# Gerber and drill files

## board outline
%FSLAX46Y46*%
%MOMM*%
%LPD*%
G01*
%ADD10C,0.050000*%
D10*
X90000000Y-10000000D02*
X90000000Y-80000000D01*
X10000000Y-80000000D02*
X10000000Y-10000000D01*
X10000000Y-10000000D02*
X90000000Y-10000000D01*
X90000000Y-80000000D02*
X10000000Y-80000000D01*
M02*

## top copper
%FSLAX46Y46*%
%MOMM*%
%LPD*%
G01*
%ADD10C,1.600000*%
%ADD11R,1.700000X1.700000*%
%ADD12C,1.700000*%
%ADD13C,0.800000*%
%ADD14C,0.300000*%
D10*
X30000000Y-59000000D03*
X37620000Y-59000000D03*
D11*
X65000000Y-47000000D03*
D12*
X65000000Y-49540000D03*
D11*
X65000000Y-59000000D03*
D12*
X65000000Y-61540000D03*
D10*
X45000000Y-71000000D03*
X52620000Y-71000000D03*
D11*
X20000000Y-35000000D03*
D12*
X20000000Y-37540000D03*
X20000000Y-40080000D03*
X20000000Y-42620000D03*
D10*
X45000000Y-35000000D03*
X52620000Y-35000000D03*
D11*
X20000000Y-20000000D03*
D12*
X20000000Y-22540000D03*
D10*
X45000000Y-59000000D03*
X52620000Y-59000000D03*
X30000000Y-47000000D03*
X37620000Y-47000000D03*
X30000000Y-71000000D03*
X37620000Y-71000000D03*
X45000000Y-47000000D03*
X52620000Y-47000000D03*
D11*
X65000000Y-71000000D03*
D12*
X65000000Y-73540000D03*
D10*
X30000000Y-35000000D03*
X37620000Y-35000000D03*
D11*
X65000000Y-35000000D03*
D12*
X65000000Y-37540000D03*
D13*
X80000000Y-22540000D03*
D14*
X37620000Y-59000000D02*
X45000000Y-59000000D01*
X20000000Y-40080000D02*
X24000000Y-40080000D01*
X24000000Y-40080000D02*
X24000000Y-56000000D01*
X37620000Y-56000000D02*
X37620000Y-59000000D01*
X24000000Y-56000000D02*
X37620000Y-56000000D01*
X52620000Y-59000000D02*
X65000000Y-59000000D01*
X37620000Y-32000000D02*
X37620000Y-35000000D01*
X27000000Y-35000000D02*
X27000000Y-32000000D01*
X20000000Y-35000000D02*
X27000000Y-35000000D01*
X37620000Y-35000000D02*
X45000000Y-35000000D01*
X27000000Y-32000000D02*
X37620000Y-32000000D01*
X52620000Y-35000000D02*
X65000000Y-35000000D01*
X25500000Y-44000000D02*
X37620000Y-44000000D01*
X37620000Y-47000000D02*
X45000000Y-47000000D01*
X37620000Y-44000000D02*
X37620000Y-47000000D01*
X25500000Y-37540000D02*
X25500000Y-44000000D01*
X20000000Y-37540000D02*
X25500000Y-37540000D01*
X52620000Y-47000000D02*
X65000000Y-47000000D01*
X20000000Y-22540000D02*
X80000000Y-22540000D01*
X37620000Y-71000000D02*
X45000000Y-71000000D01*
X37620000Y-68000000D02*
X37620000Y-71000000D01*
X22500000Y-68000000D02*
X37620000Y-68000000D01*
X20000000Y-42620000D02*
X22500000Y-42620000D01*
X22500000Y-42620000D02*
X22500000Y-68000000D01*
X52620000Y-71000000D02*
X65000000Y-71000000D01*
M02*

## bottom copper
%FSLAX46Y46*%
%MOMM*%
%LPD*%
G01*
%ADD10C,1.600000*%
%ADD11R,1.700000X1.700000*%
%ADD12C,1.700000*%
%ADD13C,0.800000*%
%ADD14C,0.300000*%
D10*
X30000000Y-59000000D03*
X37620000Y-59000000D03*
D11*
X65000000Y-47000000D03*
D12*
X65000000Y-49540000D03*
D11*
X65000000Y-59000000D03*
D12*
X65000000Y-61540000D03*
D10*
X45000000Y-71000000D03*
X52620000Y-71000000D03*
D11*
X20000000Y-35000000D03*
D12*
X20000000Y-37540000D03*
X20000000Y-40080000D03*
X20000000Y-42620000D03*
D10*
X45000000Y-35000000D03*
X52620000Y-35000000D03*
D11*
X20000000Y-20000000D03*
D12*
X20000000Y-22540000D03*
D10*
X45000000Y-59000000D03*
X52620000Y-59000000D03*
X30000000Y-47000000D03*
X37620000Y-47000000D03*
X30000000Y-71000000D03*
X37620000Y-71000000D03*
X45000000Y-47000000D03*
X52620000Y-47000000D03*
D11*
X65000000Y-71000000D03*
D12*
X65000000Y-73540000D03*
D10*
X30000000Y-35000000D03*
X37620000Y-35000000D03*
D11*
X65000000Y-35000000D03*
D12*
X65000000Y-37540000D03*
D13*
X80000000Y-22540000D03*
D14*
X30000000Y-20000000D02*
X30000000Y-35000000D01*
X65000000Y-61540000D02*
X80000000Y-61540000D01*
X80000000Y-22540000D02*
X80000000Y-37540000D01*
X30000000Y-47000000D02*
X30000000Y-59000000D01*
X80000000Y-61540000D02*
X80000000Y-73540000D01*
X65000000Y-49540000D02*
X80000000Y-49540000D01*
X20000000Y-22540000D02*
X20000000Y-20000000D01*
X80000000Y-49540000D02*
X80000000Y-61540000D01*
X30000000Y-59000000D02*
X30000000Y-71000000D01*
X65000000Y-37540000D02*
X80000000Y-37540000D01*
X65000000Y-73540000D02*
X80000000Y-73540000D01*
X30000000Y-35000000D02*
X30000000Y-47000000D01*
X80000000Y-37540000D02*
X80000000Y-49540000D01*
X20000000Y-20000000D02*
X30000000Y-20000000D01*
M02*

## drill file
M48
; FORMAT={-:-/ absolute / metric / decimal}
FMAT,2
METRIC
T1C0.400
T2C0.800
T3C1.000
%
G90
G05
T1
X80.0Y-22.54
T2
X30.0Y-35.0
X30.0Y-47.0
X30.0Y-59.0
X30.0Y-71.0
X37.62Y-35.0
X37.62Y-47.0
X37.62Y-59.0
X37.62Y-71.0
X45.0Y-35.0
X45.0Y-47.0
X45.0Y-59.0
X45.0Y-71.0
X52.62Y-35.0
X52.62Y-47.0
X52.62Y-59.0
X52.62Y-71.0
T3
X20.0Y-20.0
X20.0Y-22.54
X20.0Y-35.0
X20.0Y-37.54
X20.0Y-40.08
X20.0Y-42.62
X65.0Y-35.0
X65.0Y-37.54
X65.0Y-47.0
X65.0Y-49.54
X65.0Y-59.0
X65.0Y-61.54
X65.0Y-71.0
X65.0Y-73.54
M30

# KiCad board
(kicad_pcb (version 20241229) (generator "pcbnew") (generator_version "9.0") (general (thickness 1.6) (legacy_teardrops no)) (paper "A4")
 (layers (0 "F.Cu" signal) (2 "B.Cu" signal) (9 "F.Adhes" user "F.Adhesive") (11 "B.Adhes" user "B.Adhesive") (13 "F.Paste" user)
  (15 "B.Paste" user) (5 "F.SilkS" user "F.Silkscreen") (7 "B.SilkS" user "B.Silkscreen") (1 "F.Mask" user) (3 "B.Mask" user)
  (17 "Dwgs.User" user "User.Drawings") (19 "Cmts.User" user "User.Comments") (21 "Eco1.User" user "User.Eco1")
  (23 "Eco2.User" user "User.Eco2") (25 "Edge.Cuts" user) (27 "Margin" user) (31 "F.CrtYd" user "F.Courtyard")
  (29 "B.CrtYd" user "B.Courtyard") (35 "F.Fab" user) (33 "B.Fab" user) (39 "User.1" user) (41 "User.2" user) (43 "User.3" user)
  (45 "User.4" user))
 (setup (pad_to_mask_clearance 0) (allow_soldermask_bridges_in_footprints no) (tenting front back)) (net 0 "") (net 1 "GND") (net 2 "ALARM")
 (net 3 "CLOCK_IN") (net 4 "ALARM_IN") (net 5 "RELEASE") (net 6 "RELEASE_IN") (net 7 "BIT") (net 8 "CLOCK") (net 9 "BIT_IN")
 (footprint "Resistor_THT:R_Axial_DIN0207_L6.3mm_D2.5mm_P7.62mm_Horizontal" (layer "F.Cu") (at 30 59)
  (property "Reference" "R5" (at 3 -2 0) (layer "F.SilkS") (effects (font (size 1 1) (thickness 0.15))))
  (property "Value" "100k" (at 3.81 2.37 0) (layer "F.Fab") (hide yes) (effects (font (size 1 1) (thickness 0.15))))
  (pad "1" thru_hole circle (at 0 0) (size 1.6 1.6) (drill 0.8) (layers "*.Cu" "*.Mask") (remove_unused_layers no) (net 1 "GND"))
  (pad "2" thru_hole circle (at 7.62 0) (size 1.6 1.6) (drill 0.8) (layers "*.Cu" "*.Mask") (remove_unused_layers no) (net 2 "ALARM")))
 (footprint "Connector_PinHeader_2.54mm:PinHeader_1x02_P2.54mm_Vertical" (layer "F.Cu") (at 65 47)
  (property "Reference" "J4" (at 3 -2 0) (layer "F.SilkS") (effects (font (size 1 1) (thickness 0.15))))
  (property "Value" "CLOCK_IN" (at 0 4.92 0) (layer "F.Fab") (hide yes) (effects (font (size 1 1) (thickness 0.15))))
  (pad "1" thru_hole rect (at 0 0) (size 1.7 1.7) (drill 1) (layers "*.Cu" "*.Mask") (remove_unused_layers no) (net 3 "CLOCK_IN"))
  (pad "2" thru_hole circle (at 0 2.54) (size 1.7 1.7) (drill 1) (layers "*.Cu" "*.Mask") (remove_unused_layers no) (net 1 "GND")))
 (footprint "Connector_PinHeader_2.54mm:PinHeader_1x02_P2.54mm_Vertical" (layer "F.Cu") (at 65 59)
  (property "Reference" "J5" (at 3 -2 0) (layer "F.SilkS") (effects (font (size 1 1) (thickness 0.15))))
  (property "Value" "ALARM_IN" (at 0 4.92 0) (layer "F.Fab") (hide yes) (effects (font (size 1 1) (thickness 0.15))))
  (pad "1" thru_hole rect (at 0 0) (size 1.7 1.7) (drill 1) (layers "*.Cu" "*.Mask") (remove_unused_layers no) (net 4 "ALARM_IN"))
  (pad "2" thru_hole circle (at 0 2.54) (size 1.7 1.7) (drill 1) (layers "*.Cu" "*.Mask") (remove_unused_layers no) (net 1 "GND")))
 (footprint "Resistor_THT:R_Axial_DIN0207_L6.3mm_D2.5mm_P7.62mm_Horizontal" (layer "F.Cu") (at 45 71)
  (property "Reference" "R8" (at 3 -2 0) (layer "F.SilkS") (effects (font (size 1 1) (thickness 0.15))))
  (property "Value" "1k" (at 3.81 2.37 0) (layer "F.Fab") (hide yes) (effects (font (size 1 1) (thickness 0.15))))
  (pad "1" thru_hole circle (at 0 0) (size 1.6 1.6) (drill 0.8) (layers "*.Cu" "*.Mask") (remove_unused_layers no) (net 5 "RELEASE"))
  (pad "2" thru_hole circle (at 7.62 0) (size 1.6 1.6) (drill 0.8) (layers "*.Cu" "*.Mask") (remove_unused_layers no) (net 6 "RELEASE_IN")))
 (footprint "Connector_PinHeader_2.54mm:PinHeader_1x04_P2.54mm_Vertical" (layer "F.Cu") (at 20 35)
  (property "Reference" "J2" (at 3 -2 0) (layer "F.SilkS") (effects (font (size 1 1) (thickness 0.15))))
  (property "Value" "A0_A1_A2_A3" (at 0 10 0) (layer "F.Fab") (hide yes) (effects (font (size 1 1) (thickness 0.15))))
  (pad "1" thru_hole rect (at 0 0) (size 1.7 1.7) (drill 1) (layers "*.Cu" "*.Mask") (remove_unused_layers no) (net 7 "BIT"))
  (pad "2" thru_hole circle (at 0 2.54) (size 1.7 1.7) (drill 1) (layers "*.Cu" "*.Mask") (remove_unused_layers no) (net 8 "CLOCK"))
  (pad "3" thru_hole circle (at 0 5.08) (size 1.7 1.7) (drill 1) (layers "*.Cu" "*.Mask") (remove_unused_layers no) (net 2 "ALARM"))
  (pad "4" thru_hole circle (at 0 7.62) (size 1.7 1.7) (drill 1) (layers "*.Cu" "*.Mask") (remove_unused_layers no) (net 5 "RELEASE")))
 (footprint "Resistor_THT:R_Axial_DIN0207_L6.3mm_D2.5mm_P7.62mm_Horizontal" (layer "F.Cu") (at 45 35)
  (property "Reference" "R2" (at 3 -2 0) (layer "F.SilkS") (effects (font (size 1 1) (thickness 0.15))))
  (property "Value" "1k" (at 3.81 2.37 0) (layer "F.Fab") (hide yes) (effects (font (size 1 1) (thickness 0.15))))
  (pad "1" thru_hole circle (at 0 0) (size 1.6 1.6) (drill 0.8) (layers "*.Cu" "*.Mask") (remove_unused_layers no) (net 7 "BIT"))
  (pad "2" thru_hole circle (at 7.62 0) (size 1.6 1.6) (drill 0.8) (layers "*.Cu" "*.Mask") (remove_unused_layers no) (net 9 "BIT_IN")))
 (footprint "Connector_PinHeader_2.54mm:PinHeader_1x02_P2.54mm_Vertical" (layer "F.Cu") (at 20 20)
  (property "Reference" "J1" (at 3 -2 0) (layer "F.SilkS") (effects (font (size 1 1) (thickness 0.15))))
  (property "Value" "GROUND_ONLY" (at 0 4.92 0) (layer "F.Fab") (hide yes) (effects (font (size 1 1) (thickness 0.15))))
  (pad "1" thru_hole rect (at 0 0) (size 1.7 1.7) (drill 1) (layers "*.Cu" "*.Mask") (remove_unused_layers no) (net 1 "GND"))
  (pad "2" thru_hole circle (at 0 2.54) (size 1.7 1.7) (drill 1) (layers "*.Cu" "*.Mask") (remove_unused_layers no) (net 1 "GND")))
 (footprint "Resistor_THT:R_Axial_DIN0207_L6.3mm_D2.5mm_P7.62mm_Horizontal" (layer "F.Cu") (at 45 59)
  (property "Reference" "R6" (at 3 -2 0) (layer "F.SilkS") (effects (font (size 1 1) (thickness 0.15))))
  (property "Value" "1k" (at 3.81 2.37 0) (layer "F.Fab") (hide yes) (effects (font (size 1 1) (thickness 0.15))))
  (pad "1" thru_hole circle (at 0 0) (size 1.6 1.6) (drill 0.8) (layers "*.Cu" "*.Mask") (remove_unused_layers no) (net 2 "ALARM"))
  (pad "2" thru_hole circle (at 7.62 0) (size 1.6 1.6) (drill 0.8) (layers "*.Cu" "*.Mask") (remove_unused_layers no) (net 4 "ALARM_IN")))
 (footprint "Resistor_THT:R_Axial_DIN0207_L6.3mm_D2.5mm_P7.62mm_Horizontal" (layer "F.Cu") (at 30 47)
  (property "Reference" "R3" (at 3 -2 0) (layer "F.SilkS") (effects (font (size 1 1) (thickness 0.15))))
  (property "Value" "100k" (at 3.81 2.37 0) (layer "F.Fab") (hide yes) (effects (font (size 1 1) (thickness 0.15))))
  (pad "1" thru_hole circle (at 0 0) (size 1.6 1.6) (drill 0.8) (layers "*.Cu" "*.Mask") (remove_unused_layers no) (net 1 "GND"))
  (pad "2" thru_hole circle (at 7.62 0) (size 1.6 1.6) (drill 0.8) (layers "*.Cu" "*.Mask") (remove_unused_layers no) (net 8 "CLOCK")))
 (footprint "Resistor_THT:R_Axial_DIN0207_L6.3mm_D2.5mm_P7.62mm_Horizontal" (layer "F.Cu") (at 30 71)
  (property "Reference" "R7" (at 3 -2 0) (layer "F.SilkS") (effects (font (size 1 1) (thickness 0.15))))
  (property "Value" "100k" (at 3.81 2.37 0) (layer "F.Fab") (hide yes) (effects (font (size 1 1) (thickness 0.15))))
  (pad "1" thru_hole circle (at 0 0) (size 1.6 1.6) (drill 0.8) (layers "*.Cu" "*.Mask") (remove_unused_layers no) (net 1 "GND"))
  (pad "2" thru_hole circle (at 7.62 0) (size 1.6 1.6) (drill 0.8) (layers "*.Cu" "*.Mask") (remove_unused_layers no) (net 5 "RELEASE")))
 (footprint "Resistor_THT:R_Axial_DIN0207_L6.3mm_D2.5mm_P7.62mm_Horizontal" (layer "F.Cu") (at 45 47)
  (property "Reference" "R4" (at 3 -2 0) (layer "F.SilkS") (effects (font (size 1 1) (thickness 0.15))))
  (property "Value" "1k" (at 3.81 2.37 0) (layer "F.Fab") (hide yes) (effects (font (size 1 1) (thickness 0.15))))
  (pad "1" thru_hole circle (at 0 0) (size 1.6 1.6) (drill 0.8) (layers "*.Cu" "*.Mask") (remove_unused_layers no) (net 8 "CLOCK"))
  (pad "2" thru_hole circle (at 7.62 0) (size 1.6 1.6) (drill 0.8) (layers "*.Cu" "*.Mask") (remove_unused_layers no) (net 3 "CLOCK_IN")))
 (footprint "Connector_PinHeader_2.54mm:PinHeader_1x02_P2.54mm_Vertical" (layer "F.Cu") (at 65 71)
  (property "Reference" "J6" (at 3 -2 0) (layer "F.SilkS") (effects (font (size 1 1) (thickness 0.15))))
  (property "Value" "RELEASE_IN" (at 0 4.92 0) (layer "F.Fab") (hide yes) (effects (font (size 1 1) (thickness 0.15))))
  (pad "1" thru_hole rect (at 0 0) (size 1.7 1.7) (drill 1) (layers "*.Cu" "*.Mask") (remove_unused_layers no) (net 6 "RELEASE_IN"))
  (pad "2" thru_hole circle (at 0 2.54) (size 1.7 1.7) (drill 1) (layers "*.Cu" "*.Mask") (remove_unused_layers no) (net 1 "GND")))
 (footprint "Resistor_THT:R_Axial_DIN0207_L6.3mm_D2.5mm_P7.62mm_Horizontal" (layer "F.Cu") (at 30 35)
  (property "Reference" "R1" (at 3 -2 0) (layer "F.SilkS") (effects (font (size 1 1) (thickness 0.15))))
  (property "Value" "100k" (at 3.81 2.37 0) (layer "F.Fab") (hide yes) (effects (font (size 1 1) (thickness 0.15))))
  (pad "1" thru_hole circle (at 0 0) (size 1.6 1.6) (drill 0.8) (layers "*.Cu" "*.Mask") (remove_unused_layers no) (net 1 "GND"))
  (pad "2" thru_hole circle (at 7.62 0) (size 1.6 1.6) (drill 0.8) (layers "*.Cu" "*.Mask") (remove_unused_layers no) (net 7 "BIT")))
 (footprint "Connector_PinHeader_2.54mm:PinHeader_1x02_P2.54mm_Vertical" (layer "F.Cu") (at 65 35)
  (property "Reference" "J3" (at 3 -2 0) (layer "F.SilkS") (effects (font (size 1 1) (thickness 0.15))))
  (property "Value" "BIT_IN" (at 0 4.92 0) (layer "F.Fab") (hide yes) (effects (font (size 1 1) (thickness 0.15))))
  (pad "1" thru_hole rect (at 0 0) (size 1.7 1.7) (drill 1) (layers "*.Cu" "*.Mask") (remove_unused_layers no) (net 9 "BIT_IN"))
  (pad "2" thru_hole circle (at 0 2.54) (size 1.7 1.7) (drill 1) (layers "*.Cu" "*.Mask") (remove_unused_layers no) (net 1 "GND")))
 (gr_line (start 90 10) (end 90 80) (stroke (width 0.05) (type default)) (layer "Edge.Cuts"))
 (gr_line (start 10 80) (end 10 10) (stroke (width 0.05) (type default)) (layer "Edge.Cuts"))
 (gr_line (start 10 10) (end 90 10) (stroke (width 0.05) (type default)) (layer "Edge.Cuts"))
 (gr_line (start 90 80) (end 10 80) (stroke (width 0.05) (type default)) (layer "Edge.Cuts"))
 (segment (start 37.62 59) (end 45 59) (width 0.3) (layer "F.Cu") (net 2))
 (segment (start 20 40.08) (end 24 40.08) (width 0.3) (layer "F.Cu") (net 2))
 (segment (start 24 40.08) (end 24 56) (width 0.3) (layer "F.Cu") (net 2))
 (segment (start 37.62 56) (end 37.62 59) (width 0.3) (layer "F.Cu") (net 2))
 (segment (start 24 56) (end 37.62 56) (width 0.3) (layer "F.Cu") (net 2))
 (segment (start 52.62 59) (end 65 59) (width 0.3) (layer "F.Cu") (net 4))
 (segment (start 37.62 32) (end 37.62 35) (width 0.3) (layer "F.Cu") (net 7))
 (segment (start 27 35) (end 27 32) (width 0.3) (layer "F.Cu") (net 7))
 (segment (start 20 35) (end 27 35) (width 0.3) (layer "F.Cu") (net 7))
 (segment (start 37.62 35) (end 45 35) (width 0.3) (layer "F.Cu") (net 7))
 (segment (start 27 32) (end 37.62 32) (width 0.3) (layer "F.Cu") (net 7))
 (segment (start 52.62 35) (end 65 35) (width 0.3) (layer "F.Cu") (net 9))
 (segment (start 25.5 44) (end 37.62 44) (width 0.3) (layer "F.Cu") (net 8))
 (segment (start 37.62 47) (end 45 47) (width 0.3) (layer "F.Cu") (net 8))
 (segment (start 37.62 44) (end 37.62 47) (width 0.3) (layer "F.Cu") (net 8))
 (segment (start 25.5 37.54) (end 25.5 44) (width 0.3) (layer "F.Cu") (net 8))
 (segment (start 20 37.54) (end 25.5 37.54) (width 0.3) (layer "F.Cu") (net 8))
 (segment (start 52.62 47) (end 65 47) (width 0.3) (layer "F.Cu") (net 3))
 (segment (start 20 22.54) (end 80 22.54) (width 0.3) (layer "F.Cu") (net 1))
 (via (at 80 22.54) (size 0.8) (drill 0.4) (layers "F.Cu" "B.Cu") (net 1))
 (segment (start 30 20) (end 30 35) (width 0.3) (layer "B.Cu") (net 1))
 (segment (start 65 61.54) (end 80 61.54) (width 0.3) (layer "B.Cu") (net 1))
 (segment (start 80 22.54) (end 80 37.54) (width 0.3) (layer "B.Cu") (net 1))
 (segment (start 30 47) (end 30 59) (width 0.3) (layer "B.Cu") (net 1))
 (segment (start 80 61.54) (end 80 73.54) (width 0.3) (layer "B.Cu") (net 1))
 (segment (start 65 49.54) (end 80 49.54) (width 0.3) (layer "B.Cu") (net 1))
 (segment (start 20 22.54) (end 20 20) (width 0.3) (layer "B.Cu") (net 1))
 (segment (start 80 49.54) (end 80 61.54) (width 0.3) (layer "B.Cu") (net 1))
 (segment (start 30 59) (end 30 71) (width 0.3) (layer "B.Cu") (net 1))
 (segment (start 65 37.54) (end 80 37.54) (width 0.3) (layer "B.Cu") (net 1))
 (segment (start 65 73.54) (end 80 73.54) (width 0.3) (layer "B.Cu") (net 1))
 (segment (start 30 35) (end 30 47) (width 0.3) (layer "B.Cu") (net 1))
 (segment (start 80 37.54) (end 80 49.54) (width 0.3) (layer "B.Cu") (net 1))
 (segment (start 20 20) (end 30 20) (width 0.3) (layer "B.Cu") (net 1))
 (segment (start 37.62 71) (end 45 71) (width 0.3) (layer "F.Cu") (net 5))
 (segment (start 37.62 68) (end 37.62 71) (width 0.3) (layer "F.Cu") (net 5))
 (segment (start 22.5 68) (end 37.62 68) (width 0.3) (layer "F.Cu") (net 5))
 (segment (start 20 42.62) (end 22.5 42.62) (width 0.3) (layer "F.Cu") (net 5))
 (segment (start 22.5 42.62) (end 22.5 68) (width 0.3) (layer "F.Cu") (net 5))
 (segment (start 52.62 71) (end 65 71) (width 0.3) (layer "F.Cu") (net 6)))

